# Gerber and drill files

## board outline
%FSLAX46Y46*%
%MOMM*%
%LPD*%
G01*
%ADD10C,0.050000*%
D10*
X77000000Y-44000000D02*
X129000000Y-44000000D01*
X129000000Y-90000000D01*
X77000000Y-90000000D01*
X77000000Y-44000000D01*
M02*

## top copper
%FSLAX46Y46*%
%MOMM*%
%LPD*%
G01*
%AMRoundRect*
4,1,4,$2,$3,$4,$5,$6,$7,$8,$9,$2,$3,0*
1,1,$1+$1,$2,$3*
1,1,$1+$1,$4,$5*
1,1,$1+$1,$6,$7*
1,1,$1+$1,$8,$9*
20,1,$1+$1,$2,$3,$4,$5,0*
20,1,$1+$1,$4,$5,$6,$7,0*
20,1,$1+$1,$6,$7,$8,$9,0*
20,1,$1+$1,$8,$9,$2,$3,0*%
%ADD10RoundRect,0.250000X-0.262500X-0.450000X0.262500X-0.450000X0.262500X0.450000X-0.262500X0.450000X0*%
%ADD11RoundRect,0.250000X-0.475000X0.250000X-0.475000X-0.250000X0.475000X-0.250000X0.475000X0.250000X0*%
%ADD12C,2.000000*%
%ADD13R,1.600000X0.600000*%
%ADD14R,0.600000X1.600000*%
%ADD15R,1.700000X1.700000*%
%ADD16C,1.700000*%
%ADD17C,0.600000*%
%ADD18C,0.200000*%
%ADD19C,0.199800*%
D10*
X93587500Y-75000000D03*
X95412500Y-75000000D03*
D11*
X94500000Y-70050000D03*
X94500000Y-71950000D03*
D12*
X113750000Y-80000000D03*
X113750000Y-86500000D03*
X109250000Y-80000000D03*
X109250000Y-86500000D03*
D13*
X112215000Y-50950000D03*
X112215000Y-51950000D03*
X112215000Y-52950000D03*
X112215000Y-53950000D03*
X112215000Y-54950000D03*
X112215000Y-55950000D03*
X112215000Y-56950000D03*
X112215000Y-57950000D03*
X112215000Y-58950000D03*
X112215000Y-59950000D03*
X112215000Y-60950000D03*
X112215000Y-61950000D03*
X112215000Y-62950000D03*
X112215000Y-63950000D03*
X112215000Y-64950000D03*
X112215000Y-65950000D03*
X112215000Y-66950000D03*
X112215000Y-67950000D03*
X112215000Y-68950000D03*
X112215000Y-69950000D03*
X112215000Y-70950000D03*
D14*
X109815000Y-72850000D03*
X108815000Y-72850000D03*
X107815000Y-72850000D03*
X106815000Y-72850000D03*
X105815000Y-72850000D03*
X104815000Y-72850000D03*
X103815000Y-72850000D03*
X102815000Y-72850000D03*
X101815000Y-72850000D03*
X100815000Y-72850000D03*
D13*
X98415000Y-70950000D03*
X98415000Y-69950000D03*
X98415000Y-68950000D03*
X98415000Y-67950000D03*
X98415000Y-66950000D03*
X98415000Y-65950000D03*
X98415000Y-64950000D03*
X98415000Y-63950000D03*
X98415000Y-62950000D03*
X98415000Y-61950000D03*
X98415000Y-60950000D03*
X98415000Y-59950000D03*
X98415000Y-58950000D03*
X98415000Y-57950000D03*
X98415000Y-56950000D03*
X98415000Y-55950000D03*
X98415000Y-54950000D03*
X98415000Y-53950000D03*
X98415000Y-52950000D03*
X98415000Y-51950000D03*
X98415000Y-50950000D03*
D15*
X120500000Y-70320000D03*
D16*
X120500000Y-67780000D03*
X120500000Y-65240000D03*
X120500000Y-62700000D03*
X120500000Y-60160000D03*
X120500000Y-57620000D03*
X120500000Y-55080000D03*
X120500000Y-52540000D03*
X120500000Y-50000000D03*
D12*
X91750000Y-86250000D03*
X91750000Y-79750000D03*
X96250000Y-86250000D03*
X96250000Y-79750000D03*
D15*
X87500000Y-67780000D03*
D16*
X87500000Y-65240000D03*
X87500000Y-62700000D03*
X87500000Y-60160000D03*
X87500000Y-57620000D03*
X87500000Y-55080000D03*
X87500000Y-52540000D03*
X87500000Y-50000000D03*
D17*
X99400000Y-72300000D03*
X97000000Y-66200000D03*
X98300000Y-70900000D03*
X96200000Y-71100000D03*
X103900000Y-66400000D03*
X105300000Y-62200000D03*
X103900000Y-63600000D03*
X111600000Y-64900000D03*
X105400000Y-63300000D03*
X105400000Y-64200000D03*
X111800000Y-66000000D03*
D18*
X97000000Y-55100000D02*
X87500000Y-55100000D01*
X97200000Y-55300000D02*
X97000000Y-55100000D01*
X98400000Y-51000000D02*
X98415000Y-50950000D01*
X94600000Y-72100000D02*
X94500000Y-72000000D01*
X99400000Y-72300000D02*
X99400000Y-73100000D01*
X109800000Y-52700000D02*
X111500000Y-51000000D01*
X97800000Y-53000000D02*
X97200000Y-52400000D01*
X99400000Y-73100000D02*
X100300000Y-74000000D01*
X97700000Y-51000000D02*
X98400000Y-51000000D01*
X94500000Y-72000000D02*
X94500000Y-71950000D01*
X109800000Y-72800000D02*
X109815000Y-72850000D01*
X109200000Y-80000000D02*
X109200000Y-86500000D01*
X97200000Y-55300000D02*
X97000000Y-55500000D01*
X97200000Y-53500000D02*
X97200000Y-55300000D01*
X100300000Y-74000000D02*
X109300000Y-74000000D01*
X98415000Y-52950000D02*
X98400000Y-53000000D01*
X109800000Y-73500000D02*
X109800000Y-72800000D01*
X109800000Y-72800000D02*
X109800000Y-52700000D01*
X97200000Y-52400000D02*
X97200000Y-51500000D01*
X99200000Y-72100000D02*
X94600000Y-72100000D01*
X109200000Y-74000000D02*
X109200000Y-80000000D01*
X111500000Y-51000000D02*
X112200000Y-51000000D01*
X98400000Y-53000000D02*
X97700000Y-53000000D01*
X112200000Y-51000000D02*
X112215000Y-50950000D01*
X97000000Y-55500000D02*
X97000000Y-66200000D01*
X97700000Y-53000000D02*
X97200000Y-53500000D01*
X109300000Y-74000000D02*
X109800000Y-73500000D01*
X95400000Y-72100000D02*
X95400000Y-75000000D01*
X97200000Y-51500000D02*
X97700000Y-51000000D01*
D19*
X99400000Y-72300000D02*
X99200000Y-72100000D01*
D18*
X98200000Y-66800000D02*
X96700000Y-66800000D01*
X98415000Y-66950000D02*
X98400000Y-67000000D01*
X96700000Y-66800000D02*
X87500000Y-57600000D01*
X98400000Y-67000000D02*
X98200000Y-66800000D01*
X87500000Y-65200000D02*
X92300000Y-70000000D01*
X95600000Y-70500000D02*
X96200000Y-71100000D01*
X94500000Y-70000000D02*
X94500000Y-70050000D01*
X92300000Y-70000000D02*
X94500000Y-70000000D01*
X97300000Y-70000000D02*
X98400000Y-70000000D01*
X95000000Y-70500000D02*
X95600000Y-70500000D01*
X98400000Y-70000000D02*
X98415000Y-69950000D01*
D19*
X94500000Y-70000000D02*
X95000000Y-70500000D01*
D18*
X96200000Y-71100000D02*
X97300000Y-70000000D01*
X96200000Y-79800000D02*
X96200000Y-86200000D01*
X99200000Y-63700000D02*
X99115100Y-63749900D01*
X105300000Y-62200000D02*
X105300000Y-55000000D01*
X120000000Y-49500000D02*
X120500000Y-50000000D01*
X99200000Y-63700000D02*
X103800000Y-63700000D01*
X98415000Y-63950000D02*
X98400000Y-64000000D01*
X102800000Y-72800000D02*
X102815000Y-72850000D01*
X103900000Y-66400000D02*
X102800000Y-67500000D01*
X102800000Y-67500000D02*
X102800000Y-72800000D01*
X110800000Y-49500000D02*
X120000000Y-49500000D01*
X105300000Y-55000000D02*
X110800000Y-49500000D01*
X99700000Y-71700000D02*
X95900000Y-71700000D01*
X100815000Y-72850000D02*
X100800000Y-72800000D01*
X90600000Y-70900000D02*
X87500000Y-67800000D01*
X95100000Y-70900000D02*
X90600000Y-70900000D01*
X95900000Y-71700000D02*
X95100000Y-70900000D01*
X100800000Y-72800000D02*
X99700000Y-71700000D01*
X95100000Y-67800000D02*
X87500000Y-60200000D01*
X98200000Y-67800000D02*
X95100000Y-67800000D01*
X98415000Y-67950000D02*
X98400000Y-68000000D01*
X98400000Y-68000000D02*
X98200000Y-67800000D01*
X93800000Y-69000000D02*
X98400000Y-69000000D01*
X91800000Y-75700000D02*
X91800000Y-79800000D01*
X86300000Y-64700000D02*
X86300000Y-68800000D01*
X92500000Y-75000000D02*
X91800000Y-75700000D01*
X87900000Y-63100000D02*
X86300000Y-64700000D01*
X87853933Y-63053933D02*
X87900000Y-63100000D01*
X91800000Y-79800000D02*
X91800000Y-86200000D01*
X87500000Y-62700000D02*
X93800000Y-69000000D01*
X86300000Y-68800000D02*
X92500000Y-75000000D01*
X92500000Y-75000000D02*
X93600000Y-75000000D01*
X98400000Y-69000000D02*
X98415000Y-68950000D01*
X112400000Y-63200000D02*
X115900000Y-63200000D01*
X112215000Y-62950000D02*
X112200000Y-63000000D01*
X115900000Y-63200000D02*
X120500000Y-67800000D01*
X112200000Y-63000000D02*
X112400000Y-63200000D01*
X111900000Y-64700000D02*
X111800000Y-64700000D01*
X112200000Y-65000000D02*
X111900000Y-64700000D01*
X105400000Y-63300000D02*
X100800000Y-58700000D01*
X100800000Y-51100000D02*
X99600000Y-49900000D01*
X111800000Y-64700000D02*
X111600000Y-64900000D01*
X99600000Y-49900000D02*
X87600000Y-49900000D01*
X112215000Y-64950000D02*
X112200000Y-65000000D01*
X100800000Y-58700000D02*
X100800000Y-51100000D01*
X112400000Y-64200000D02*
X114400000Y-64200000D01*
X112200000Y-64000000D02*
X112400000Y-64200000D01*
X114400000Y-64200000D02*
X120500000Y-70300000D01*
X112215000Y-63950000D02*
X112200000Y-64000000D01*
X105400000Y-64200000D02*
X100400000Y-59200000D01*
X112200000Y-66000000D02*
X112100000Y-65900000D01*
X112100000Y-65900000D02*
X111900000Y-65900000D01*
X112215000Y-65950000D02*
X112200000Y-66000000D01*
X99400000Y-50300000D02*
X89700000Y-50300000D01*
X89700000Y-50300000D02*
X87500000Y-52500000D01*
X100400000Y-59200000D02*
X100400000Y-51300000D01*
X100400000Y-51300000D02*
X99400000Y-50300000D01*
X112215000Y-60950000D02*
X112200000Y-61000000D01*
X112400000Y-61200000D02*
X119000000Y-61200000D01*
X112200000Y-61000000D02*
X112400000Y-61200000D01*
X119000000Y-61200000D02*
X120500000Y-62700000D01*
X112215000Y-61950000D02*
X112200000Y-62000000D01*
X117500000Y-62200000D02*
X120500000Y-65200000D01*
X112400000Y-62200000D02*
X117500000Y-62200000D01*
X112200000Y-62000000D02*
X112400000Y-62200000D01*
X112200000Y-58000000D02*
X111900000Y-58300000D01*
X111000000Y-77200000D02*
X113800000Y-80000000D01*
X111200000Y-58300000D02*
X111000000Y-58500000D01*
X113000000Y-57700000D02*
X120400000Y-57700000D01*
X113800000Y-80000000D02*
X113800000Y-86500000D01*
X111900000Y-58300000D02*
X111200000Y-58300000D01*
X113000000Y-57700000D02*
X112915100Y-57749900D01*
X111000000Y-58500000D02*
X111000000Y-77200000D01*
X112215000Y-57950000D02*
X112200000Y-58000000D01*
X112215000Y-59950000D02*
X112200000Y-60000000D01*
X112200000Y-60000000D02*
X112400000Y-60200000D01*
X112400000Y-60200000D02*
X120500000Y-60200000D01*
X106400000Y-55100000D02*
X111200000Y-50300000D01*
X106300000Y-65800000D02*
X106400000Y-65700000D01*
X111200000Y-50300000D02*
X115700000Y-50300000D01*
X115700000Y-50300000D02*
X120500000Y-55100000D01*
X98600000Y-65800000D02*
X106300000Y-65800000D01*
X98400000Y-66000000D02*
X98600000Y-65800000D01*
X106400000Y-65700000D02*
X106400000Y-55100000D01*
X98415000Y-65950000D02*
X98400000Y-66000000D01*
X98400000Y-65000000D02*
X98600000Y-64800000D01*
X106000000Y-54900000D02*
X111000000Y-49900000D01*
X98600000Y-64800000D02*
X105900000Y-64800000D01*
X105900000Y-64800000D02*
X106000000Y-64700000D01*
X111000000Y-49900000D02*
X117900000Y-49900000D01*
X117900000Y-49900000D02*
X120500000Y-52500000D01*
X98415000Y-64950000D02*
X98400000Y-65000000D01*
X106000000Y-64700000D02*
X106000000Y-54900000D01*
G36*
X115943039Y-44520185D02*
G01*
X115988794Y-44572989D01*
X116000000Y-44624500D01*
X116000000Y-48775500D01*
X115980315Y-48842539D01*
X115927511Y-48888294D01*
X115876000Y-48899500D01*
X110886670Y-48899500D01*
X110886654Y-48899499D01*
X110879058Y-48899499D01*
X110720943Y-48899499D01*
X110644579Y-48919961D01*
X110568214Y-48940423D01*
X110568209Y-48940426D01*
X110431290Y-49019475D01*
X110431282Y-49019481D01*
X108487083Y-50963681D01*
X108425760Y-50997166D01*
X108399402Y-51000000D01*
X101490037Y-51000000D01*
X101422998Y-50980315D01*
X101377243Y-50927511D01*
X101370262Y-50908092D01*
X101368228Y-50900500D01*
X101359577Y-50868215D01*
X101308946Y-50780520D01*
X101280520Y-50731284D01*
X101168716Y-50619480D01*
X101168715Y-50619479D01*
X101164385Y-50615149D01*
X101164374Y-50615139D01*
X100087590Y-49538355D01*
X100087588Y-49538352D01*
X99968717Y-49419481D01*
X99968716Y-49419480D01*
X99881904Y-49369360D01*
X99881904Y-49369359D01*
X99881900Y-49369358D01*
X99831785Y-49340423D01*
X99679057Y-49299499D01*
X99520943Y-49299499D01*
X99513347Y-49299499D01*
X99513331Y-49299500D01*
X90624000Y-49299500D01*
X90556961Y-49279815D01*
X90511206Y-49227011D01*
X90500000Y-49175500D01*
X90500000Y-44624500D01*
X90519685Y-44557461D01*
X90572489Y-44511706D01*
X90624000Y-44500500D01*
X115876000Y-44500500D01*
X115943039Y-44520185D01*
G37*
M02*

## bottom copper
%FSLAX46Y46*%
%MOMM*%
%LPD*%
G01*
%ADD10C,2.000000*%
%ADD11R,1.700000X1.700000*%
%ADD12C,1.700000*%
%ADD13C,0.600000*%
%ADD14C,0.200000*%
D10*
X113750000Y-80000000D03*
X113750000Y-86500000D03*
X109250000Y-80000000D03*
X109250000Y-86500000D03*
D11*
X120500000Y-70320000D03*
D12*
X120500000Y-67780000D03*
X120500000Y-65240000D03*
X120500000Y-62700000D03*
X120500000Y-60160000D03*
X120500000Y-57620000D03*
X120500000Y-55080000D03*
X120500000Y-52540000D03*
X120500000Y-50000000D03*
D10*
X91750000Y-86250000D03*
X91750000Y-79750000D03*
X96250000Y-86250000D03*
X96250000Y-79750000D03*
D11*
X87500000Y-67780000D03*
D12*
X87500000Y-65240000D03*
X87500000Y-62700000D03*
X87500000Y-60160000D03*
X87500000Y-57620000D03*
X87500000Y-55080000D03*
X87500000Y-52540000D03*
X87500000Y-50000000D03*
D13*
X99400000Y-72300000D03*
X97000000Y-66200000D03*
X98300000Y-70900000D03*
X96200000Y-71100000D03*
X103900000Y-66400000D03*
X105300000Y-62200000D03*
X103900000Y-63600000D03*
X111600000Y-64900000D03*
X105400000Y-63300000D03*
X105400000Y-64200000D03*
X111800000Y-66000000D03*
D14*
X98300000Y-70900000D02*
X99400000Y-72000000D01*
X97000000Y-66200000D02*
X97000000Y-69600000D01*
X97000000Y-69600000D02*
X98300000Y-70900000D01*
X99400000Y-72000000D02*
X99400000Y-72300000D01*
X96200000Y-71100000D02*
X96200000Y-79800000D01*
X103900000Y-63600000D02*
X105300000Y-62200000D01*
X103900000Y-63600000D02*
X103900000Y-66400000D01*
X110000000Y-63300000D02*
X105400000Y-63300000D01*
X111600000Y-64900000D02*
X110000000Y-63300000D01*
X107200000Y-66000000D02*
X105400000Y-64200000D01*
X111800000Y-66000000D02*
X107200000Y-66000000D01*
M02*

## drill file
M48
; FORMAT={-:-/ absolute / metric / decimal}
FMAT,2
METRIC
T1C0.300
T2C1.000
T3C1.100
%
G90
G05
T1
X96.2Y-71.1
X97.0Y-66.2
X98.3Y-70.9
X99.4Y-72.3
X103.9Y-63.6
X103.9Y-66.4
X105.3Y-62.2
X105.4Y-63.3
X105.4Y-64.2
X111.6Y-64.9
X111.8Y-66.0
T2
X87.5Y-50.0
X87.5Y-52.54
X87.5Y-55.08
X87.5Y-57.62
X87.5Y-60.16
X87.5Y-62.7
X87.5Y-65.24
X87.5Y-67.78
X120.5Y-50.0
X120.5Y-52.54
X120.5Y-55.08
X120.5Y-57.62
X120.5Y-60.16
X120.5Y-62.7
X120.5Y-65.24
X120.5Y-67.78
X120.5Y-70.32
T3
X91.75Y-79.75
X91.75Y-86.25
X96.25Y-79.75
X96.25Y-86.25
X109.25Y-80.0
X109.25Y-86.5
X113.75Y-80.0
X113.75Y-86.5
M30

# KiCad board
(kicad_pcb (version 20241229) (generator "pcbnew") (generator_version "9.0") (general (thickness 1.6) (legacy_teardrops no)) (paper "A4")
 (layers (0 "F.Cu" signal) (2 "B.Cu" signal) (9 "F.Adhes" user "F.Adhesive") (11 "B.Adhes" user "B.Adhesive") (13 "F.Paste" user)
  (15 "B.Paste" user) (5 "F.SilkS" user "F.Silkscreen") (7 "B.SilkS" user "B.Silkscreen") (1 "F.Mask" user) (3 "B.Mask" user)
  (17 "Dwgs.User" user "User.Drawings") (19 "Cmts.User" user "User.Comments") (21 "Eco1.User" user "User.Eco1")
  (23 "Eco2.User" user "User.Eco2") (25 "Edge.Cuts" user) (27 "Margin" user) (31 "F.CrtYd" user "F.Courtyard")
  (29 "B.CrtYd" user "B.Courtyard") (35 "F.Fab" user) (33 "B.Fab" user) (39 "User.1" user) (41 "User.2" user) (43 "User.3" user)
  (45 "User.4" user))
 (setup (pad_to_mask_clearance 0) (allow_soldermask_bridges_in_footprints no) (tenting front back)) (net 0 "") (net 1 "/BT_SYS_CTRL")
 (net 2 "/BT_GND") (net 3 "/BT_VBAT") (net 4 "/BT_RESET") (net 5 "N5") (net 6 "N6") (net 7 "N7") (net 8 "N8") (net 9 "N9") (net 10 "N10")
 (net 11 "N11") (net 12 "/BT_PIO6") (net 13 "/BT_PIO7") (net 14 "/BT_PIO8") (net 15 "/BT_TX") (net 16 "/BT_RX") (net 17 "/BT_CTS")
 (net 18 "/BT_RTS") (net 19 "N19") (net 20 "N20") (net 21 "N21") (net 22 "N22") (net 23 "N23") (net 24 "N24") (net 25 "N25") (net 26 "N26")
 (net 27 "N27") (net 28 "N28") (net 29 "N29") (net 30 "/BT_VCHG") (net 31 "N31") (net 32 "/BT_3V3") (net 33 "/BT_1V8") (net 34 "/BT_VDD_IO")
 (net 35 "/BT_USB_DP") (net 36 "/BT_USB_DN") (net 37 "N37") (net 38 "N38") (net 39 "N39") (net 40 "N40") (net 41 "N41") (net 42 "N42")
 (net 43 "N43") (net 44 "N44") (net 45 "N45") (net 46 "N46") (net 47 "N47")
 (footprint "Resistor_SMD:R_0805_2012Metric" (layer "F.Cu") (at 94.5 75)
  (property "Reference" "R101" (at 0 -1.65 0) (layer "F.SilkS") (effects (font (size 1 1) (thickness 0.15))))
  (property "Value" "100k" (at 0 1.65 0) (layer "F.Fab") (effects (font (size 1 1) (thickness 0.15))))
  (pad "1" smd roundrect (at -0.9125 0) (size 1.025 1.4) (layers "F.Cu" "F.Mask" "F.Paste") (roundrect_rratio 0.243902)
   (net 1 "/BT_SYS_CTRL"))
  (pad "2" smd roundrect (at 0.9125 0) (size 1.025 1.4) (layers "F.Cu" "F.Mask" "F.Paste") (roundrect_rratio 0.243902) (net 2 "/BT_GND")))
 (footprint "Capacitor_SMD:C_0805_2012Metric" (layer "F.Cu") (at 94.5 71 -90)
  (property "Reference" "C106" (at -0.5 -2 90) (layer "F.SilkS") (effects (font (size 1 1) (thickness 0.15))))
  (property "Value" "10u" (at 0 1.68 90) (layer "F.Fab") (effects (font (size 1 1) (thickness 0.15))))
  (pad "1" smd roundrect (at -0.95 0 270) (size 1 1.45) (layers "F.Cu" "F.Mask" "F.Paste") (roundrect_rratio 0.25) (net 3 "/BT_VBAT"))
  (pad "2" smd roundrect (at 0.95 0 270) (size 1 1.45) (layers "F.Cu" "F.Mask" "F.Paste") (roundrect_rratio 0.25) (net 2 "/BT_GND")))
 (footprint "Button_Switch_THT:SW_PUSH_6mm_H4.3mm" (layer "F.Cu") (at 113.75 80 -90)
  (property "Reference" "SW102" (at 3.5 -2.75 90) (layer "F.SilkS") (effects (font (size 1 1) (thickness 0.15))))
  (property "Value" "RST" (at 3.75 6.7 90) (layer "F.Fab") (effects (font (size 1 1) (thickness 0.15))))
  (pad "1" thru_hole circle (at 0 0) (size 2 2) (drill 1.1) (layers "*.Cu" "*.Mask") (remove_unused_layers no) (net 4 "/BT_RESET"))
  (pad "1" thru_hole circle (at 6.5 0) (size 2 2) (drill 1.1) (layers "*.Cu" "*.Mask") (remove_unused_layers no) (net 4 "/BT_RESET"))
  (pad "2" thru_hole circle (at 0 4.5) (size 2 2) (drill 1.1) (layers "*.Cu" "*.Mask") (remove_unused_layers no) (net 2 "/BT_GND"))
  (pad "2" thru_hole circle (at 6.5 4.5) (size 2 2) (drill 1.1) (layers "*.Cu" "*.Mask") (remove_unused_layers no) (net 2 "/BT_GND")))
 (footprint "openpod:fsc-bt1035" (layer "F.Cu") (at 105.315 59 180)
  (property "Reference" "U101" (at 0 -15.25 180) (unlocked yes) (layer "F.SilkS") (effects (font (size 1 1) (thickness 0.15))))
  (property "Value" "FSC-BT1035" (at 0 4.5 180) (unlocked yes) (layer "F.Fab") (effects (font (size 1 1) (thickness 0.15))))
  (pad "1" smd rect (at -6.9 8.05 180) (size 1.6 0.6) (layers "F.Cu" "F.Mask" "F.Paste") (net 2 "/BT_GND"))
  (pad "2" smd rect (at -6.9 7.05 180) (size 1.6 0.6) (layers "F.Cu" "F.Mask" "F.Paste") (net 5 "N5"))
  (pad "3" smd rect (at -6.9 6.05 180) (size 1.6 0.6) (layers "F.Cu" "F.Mask" "F.Paste") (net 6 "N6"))
  (pad "4" smd rect (at -6.9 5.05 180) (size 1.6 0.6) (layers "F.Cu" "F.Mask" "F.Paste") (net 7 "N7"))
  (pad "5" smd rect (at -6.9 4.05 180) (size 1.6 0.6) (layers "F.Cu" "F.Mask" "F.Paste") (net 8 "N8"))
  (pad "6" smd rect (at -6.9 3.05 180) (size 1.6 0.6) (layers "F.Cu" "F.Mask" "F.Paste") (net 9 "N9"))
  (pad "7" smd rect (at -6.9 2.05 180) (size 1.6 0.6) (layers "F.Cu" "F.Mask" "F.Paste") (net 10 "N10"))
  (pad "8" smd rect (at -6.9 1.05 180) (size 1.6 0.6) (layers "F.Cu" "F.Mask" "F.Paste") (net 4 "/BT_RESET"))
  (pad "9" smd rect (at -6.9 0.05 180) (size 1.6 0.6) (layers "F.Cu" "F.Mask" "F.Paste") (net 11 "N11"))
  (pad "10" smd rect (at -6.9 -0.95 180) (size 1.6 0.6) (layers "F.Cu" "F.Mask" "F.Paste") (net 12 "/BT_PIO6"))
  (pad "11" smd rect (at -6.9 -1.95 180) (size 1.6 0.6) (layers "F.Cu" "F.Mask" "F.Paste") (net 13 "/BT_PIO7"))
  (pad "12" smd rect (at -6.9 -2.95 180) (size 1.6 0.6) (layers "F.Cu" "F.Mask" "F.Paste") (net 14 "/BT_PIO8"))
  (pad "13" smd rect (at -6.9 -3.95 180) (size 1.6 0.6) (layers "F.Cu" "F.Mask" "F.Paste") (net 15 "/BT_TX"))
  (pad "14" smd rect (at -6.9 -4.95 180) (size 1.6 0.6) (layers "F.Cu" "F.Mask" "F.Paste") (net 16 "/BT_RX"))
  (pad "15" smd rect (at -6.9 -5.95 180) (size 1.6 0.6) (layers "F.Cu" "F.Mask" "F.Paste") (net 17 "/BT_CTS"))
  (pad "16" smd rect (at -6.9 -6.95 180) (size 1.6 0.6) (layers "F.Cu" "F.Mask" "F.Paste") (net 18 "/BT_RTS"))
  (pad "17" smd rect (at -6.9 -7.95 180) (size 1.6 0.6) (layers "F.Cu" "F.Mask" "F.Paste") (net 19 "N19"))
  (pad "18" smd rect (at -6.9 -8.95 180) (size 1.6 0.6) (layers "F.Cu" "F.Mask" "F.Paste") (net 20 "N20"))
  (pad "19" smd rect (at -6.9 -9.95 180) (size 1.6 0.6) (layers "F.Cu" "F.Mask" "F.Paste") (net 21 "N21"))
  (pad "20" smd rect (at -6.9 -10.95 180) (size 1.6 0.6) (layers "F.Cu" "F.Mask" "F.Paste") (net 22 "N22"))
  (pad "21" smd rect (at -6.9 -11.95 180) (size 1.6 0.6) (layers "F.Cu" "F.Mask" "F.Paste") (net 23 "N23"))
  (pad "22" smd rect (at -4.5 -13.85 180) (size 0.6 1.6) (layers "F.Cu" "F.Mask" "F.Paste") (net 2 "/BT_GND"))
  (pad "23" smd rect (at -3.5 -13.85 180) (size 0.6 1.6) (layers "F.Cu" "F.Mask" "F.Paste") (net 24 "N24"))
  (pad "24" smd rect (at -2.5 -13.85 180) (size 0.6 1.6) (layers "F.Cu" "F.Mask" "F.Paste") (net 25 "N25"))
  (pad "25" smd rect (at -1.5 -13.85 180) (size 0.6 1.6) (layers "F.Cu" "F.Mask" "F.Paste") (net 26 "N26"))
  (pad "26" smd rect (at -0.5 -13.85 180) (size 0.6 1.6) (layers "F.Cu" "F.Mask" "F.Paste") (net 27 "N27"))
  (pad "27" smd rect (at 0.5 -13.85 180) (size 0.6 1.6) (layers "F.Cu" "F.Mask" "F.Paste") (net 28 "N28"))
  (pad "28" smd rect (at 1.5 -13.85 180) (size 0.6 1.6) (layers "F.Cu" "F.Mask" "F.Paste") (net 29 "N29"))
  (pad "29" smd rect (at 2.5 -13.85 180) (size 0.6 1.6) (layers "F.Cu" "F.Mask" "F.Paste") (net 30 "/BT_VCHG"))
  (pad "30" smd rect (at 3.5 -13.85 180) (size 0.6 1.6) (layers "F.Cu" "F.Mask" "F.Paste") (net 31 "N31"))
  (pad "31" smd rect (at 4.5 -13.85 180) (size 0.6 1.6) (layers "F.Cu" "F.Mask" "F.Paste") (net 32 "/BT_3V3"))
  (pad "32" smd rect (at 6.9 -11.95 180) (size 1.6 0.6) (layers "F.Cu" "F.Mask" "F.Paste") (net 2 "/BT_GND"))
  (pad "33" smd rect (at 6.9 -10.95 180) (size 1.6 0.6) (layers "F.Cu" "F.Mask" "F.Paste") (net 3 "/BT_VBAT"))
  (pad "34" smd rect (at 6.9 -9.95 180) (size 1.6 0.6) (layers "F.Cu" "F.Mask" "F.Paste") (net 1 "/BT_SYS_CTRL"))
  (pad "35" smd rect (at 6.9 -8.95 180) (size 1.6 0.6) (layers "F.Cu" "F.Mask" "F.Paste") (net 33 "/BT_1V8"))
  (pad "36" smd rect (at 6.9 -7.95 180) (size 1.6 0.6) (layers "F.Cu" "F.Mask" "F.Paste") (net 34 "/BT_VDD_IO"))
  (pad "37" smd rect (at 6.9 -6.95 180) (size 1.6 0.6) (layers "F.Cu" "F.Mask" "F.Paste") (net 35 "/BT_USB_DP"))
  (pad "38" smd rect (at 6.9 -5.95 180) (size 1.6 0.6) (layers "F.Cu" "F.Mask" "F.Paste") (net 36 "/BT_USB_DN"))
  (pad "39" smd rect (at 6.9 -4.95 180) (size 1.6 0.6) (layers "F.Cu" "F.Mask" "F.Paste") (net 30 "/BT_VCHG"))
  (pad "40" smd rect (at 6.9 -3.95 180) (size 1.6 0.6) (layers "F.Cu" "F.Mask" "F.Paste") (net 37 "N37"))
  (pad "41" smd rect (at 6.9 -2.95 180) (size 1.6 0.6) (layers "F.Cu" "F.Mask" "F.Paste") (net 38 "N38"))
  (pad "42" smd rect (at 6.9 -1.95 180) (size 1.6 0.6) (layers "F.Cu" "F.Mask" "F.Paste") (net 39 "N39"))
  (pad "43" smd rect (at 6.9 -0.95 180) (size 1.6 0.6) (layers "F.Cu" "F.Mask" "F.Paste") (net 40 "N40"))
  (pad "44" smd rect (at 6.9 0.05 180) (size 1.6 0.6) (layers "F.Cu" "F.Mask" "F.Paste") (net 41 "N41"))
  (pad "45" smd rect (at 6.9 1.05 180) (size 1.6 0.6) (layers "F.Cu" "F.Mask" "F.Paste") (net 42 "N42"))
  (pad "46" smd rect (at 6.9 2.05 180) (size 1.6 0.6) (layers "F.Cu" "F.Mask" "F.Paste") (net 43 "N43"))
  (pad "47" smd rect (at 6.9 3.05 180) (size 1.6 0.6) (layers "F.Cu" "F.Mask" "F.Paste") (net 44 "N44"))
  (pad "48" smd rect (at 6.9 4.05 180) (size 1.6 0.6) (layers "F.Cu" "F.Mask" "F.Paste") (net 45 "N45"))
  (pad "49" smd rect (at 6.9 5.05 180) (size 1.6 0.6) (layers "F.Cu" "F.Mask" "F.Paste") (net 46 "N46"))
  (pad "50" smd rect (at 6.9 6.05 180) (size 1.6 0.6) (layers "F.Cu" "F.Mask" "F.Paste") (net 2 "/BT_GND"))
  (pad "51" smd rect (at 6.9 7.05 180) (size 1.6 0.6) (layers "F.Cu" "F.Mask" "F.Paste") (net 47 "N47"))
  (pad "52" smd rect (at 6.9 8.05 180) (size 1.6 0.6) (layers "F.Cu" "F.Mask" "F.Paste") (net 2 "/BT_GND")))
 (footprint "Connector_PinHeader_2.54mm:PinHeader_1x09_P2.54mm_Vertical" (layer "F.Cu") (at 120.5 70.32 180)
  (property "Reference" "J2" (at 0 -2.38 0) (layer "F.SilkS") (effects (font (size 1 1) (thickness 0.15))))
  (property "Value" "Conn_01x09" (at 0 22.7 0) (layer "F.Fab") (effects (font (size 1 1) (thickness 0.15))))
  (pad "1" thru_hole rect (at 0 0 180) (size 1.7 1.7) (drill 1) (layers "*.Cu" "*.Mask") (remove_unused_layers no) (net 16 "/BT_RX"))
  (pad "2" thru_hole circle (at 0 2.54 180) (size 1.7 1.7) (drill 1) (layers "*.Cu" "*.Mask") (remove_unused_layers no) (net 15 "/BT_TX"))
  (pad "3" thru_hole circle (at 0 5.08 180) (size 1.7 1.7) (drill 1) (layers "*.Cu" "*.Mask") (remove_unused_layers no) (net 14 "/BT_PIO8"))
  (pad "4" thru_hole circle (at 0 7.62 180) (size 1.7 1.7) (drill 1) (layers "*.Cu" "*.Mask") (remove_unused_layers no) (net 13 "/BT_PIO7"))
  (pad "5" thru_hole circle (at 0 10.16 180) (size 1.7 1.7) (drill 1) (layers "*.Cu" "*.Mask") (remove_unused_layers no) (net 12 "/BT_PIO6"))
  (pad "6" thru_hole circle (at 0 12.7 180) (size 1.7 1.7) (drill 1) (layers "*.Cu" "*.Mask") (remove_unused_layers no) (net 4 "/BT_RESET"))
  (pad "7" thru_hole circle (at 0 15.24 180) (size 1.7 1.7) (drill 1) (layers "*.Cu" "*.Mask") (remove_unused_layers no)
   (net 35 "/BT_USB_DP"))
  (pad "8" thru_hole circle (at 0 17.78 180) (size 1.7 1.7) (drill 1) (layers "*.Cu" "*.Mask") (remove_unused_layers no)
   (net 36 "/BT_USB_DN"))
  (pad "9" thru_hole circle (at 0 20.32 180) (size 1.7 1.7) (drill 1) (layers "*.Cu" "*.Mask") (remove_unused_layers no) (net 30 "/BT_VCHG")))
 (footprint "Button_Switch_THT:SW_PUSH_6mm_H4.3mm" (layer "F.Cu") (at 91.75 86.25 90)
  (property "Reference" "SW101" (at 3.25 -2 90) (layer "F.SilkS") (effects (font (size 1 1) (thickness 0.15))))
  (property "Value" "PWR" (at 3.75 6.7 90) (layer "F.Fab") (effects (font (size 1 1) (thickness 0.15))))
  (pad "1" thru_hole circle (at 0 0 180) (size 2 2) (drill 1.1) (layers "*.Cu" "*.Mask") (remove_unused_layers no) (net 1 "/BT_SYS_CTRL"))
  (pad "1" thru_hole circle (at 6.5 0 180) (size 2 2) (drill 1.1) (layers "*.Cu" "*.Mask") (remove_unused_layers no) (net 1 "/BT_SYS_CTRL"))
  (pad "2" thru_hole circle (at 0 4.5 180) (size 2 2) (drill 1.1) (layers "*.Cu" "*.Mask") (remove_unused_layers no) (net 3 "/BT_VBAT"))
  (pad "2" thru_hole circle (at 6.5 4.5 180) (size 2 2) (drill 1.1) (layers "*.Cu" "*.Mask") (remove_unused_layers no) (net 3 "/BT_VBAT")))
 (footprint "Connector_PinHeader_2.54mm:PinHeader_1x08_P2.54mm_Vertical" (layer "F.Cu") (at 87.5 67.78 180)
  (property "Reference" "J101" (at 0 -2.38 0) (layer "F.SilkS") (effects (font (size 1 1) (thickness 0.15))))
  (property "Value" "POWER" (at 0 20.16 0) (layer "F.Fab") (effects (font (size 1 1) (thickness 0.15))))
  (pad "1" thru_hole rect (at 0 0 180) (size 1.7 1.7) (drill 1) (layers "*.Cu" "*.Mask") (remove_unused_layers no) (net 32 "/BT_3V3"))
  (pad "2" thru_hole circle (at 0 2.54 180) (size 1.7 1.7) (drill 1) (layers "*.Cu" "*.Mask") (remove_unused_layers no) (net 3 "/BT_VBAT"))
  (pad "3" thru_hole circle (at 0 5.08 180) (size 1.7 1.7) (drill 1) (layers "*.Cu" "*.Mask") (remove_unused_layers no)
   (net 1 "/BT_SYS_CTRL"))
  (pad "4" thru_hole circle (at 0 7.62 180) (size 1.7 1.7) (drill 1) (layers "*.Cu" "*.Mask") (remove_unused_layers no) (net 33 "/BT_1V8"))
  (pad "5" thru_hole circle (at 0 10.16 180) (size 1.7 1.7) (drill 1) (layers "*.Cu" "*.Mask") (remove_unused_layers no)
   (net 34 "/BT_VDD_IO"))
  (pad "6" thru_hole circle (at 0 12.7 180) (size 1.7 1.7) (drill 1) (layers "*.Cu" "*.Mask") (remove_unused_layers no) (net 2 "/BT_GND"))
  (pad "7" thru_hole circle (at 0 15.24 180) (size 1.7 1.7) (drill 1) (layers "*.Cu" "*.Mask") (remove_unused_layers no) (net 18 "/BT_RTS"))
  (pad "8" thru_hole circle (at 0 17.78 180) (size 1.7 1.7) (drill 1) (layers "*.Cu" "*.Mask") (remove_unused_layers no) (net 17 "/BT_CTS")))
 (gr_rect (start 77 44) (end 129 90) (stroke (width 0.05) (type default)) (fill no) (layer "Edge.Cuts"))
 (segment (start 97 55.1) (end 87.5 55.1) (width 0.2) (layer "F.Cu") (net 2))
 (segment (start 97.2 55.3) (end 97 55.1) (width 0.2) (layer "F.Cu") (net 2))
 (segment (start 98.4 51) (end 98.415 50.95) (width 0.2) (layer "F.Cu") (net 2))
 (segment (start 94.6 72.1) (end 94.5 72) (width 0.2) (layer "F.Cu") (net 2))
 (segment (start 99.4 72.3) (end 99.4 73.1) (width 0.2) (layer "F.Cu") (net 2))
 (segment (start 109.8 52.7) (end 111.5 51) (width 0.2) (layer "F.Cu") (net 2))
 (segment (start 97.8 53) (end 97.2 52.4) (width 0.2) (layer "F.Cu") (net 2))
 (segment (start 99.4 73.1) (end 100.3 74) (width 0.2) (layer "F.Cu") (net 2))
 (segment (start 97.7 51) (end 98.4 51) (width 0.2) (layer "F.Cu") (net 2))
 (segment (start 94.5 72) (end 94.5 71.95) (width 0.2) (layer "F.Cu") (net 2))
 (segment (start 109.8 72.8) (end 109.815 72.85) (width 0.2) (layer "F.Cu") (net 2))
 (segment (start 109.2 80) (end 109.2 86.5) (width 0.2) (layer "F.Cu") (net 2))
 (segment (start 97.2 55.3) (end 97 55.5) (width 0.2) (layer "F.Cu") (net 2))
 (segment (start 97.2 53.5) (end 97.2 55.3) (width 0.2) (layer "F.Cu") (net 2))
 (segment (start 100.3 74) (end 109.3 74) (width 0.2) (layer "F.Cu") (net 2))
 (segment (start 98.415 52.95) (end 98.4 53) (width 0.2) (layer "F.Cu") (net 2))
 (segment (start 109.8 73.5) (end 109.8 72.8) (width 0.2) (layer "F.Cu") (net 2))
 (segment (start 109.8 72.8) (end 109.8 52.7) (width 0.2) (layer "F.Cu") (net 2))
 (segment (start 97.2 52.4) (end 97.2 51.5) (width 0.2) (layer "F.Cu") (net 2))
 (segment (start 99.2 72.1) (end 94.6 72.1) (width 0.2) (layer "F.Cu") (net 2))
 (segment (start 109.2 74) (end 109.2 80) (width 0.2) (layer "F.Cu") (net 2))
 (segment (start 111.5 51) (end 112.2 51) (width 0.2) (layer "F.Cu") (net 2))
 (segment (start 98.4 53) (end 97.7 53) (width 0.2) (layer "F.Cu") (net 2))
 (segment (start 112.2 51) (end 112.215 50.95) (width 0.2) (layer "F.Cu") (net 2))
 (segment (start 97 55.5) (end 97 66.2) (width 0.2) (layer "F.Cu") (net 2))
 (segment (start 97.7 53) (end 97.2 53.5) (width 0.2) (layer "F.Cu") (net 2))
 (segment (start 109.3 74) (end 109.8 73.5) (width 0.2) (layer "F.Cu") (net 2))
 (segment (start 95.4 72.1) (end 95.4 75) (width 0.2) (layer "F.Cu") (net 2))
 (segment (start 97.2 51.5) (end 97.7 51) (width 0.2) (layer "F.Cu") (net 2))
 (segment (start 99.4 72.3) (end 99.2 72.1) (width 0.1998) (layer "F.Cu") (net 2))
 (via (at 99.4 72.3) (size 0.6) (drill 0.3) (layers "F.Cu" "B.Cu") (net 2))
 (via (at 97 66.2) (size 0.6) (drill 0.3) (layers "F.Cu" "B.Cu") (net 2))
 (via (at 98.3 70.9) (size 0.6) (drill 0.3) (layers "F.Cu" "B.Cu") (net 2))
 (segment (start 98.3 70.9) (end 99.4 72) (width 0.2) (layer "B.Cu") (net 2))
 (segment (start 97 66.2) (end 97 69.6) (width 0.2) (layer "B.Cu") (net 2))
 (segment (start 97 69.6) (end 98.3 70.9) (width 0.2) (layer "B.Cu") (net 2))
 (segment (start 99.4 72) (end 99.4 72.3) (width 0.2) (layer "B.Cu") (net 2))
 (segment (start 98.2 66.8) (end 96.7 66.8) (width 0.2) (layer "F.Cu") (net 34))
 (segment (start 98.415 66.95) (end 98.4 67) (width 0.2) (layer "F.Cu") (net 34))
 (segment (start 96.7 66.8) (end 87.5 57.6) (width 0.2) (layer "F.Cu") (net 34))
 (segment (start 98.4 67) (end 98.2 66.8) (width 0.2) (layer "F.Cu") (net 34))
 (segment (start 87.5 65.2) (end 92.3 70) (width 0.2) (layer "F.Cu") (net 3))
 (segment (start 95.6 70.5) (end 96.2 71.1) (width 0.2) (layer "F.Cu") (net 3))
 (segment (start 94.5 70) (end 94.5 70.05) (width 0.2) (layer "F.Cu") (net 3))
 (segment (start 92.3 70) (end 94.5 70) (width 0.2) (layer "F.Cu") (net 3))
 (segment (start 97.3 70) (end 98.4 70) (width 0.2) (layer "F.Cu") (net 3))
 (segment (start 95 70.5) (end 95.6 70.5) (width 0.2) (layer "F.Cu") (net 3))
 (segment (start 98.4 70) (end 98.415 69.95) (width 0.2) (layer "F.Cu") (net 3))
 (segment (start 94.5 70) (end 95 70.5) (width 0.1998) (layer "F.Cu") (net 3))
 (segment (start 96.2 71.1) (end 97.3 70) (width 0.2) (layer "F.Cu") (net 3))
 (segment (start 96.2 79.8) (end 96.2 86.2) (width 0.2) (layer "F.Cu") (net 3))
 (via (at 96.2 71.1) (size 0.6) (drill 0.3) (layers "F.Cu" "B.Cu") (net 3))
 (segment (start 96.2 71.1) (end 96.2 79.8) (width 0.2) (layer "B.Cu") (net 3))
 (segment (start 99.2 63.7) (end 99.1151 63.7499) (width 0.2) (layer "F.Cu") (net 30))
 (segment (start 105.3 62.2) (end 105.3 55) (width 0.2) (layer "F.Cu") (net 30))
 (segment (start 120 49.5) (end 120.5 50) (width 0.2) (layer "F.Cu") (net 30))
 (segment (start 99.2 63.7) (end 103.8 63.7) (width 0.2) (layer "F.Cu") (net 30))
 (segment (start 98.415 63.95) (end 98.4 64) (width 0.2) (layer "F.Cu") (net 30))
 (segment (start 102.8 72.8) (end 102.815 72.85) (width 0.2) (layer "F.Cu") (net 30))
 (segment (start 103.9 66.4) (end 102.8 67.5) (width 0.2) (layer "F.Cu") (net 30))
 (segment (start 102.8 67.5) (end 102.8 72.8) (width 0.2) (layer "F.Cu") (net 30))
 (segment (start 110.8 49.5) (end 120 49.5) (width 0.2) (layer "F.Cu") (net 30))
 (segment (start 105.3 55) (end 110.8 49.5) (width 0.2) (layer "F.Cu") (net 30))
 (via (at 103.9 66.4) (size 0.6) (drill 0.3) (layers "F.Cu" "B.Cu") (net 30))
 (via (at 105.3 62.2) (size 0.6) (drill 0.3) (layers "F.Cu" "B.Cu") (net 30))
 (via (at 103.9 63.6) (size 0.6) (drill 0.3) (layers "F.Cu" "B.Cu") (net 30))
 (segment (start 103.9 63.6) (end 105.3 62.2) (width 0.2) (layer "B.Cu") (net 30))
 (segment (start 103.9 63.6) (end 103.9 66.4) (width 0.2) (layer "B.Cu") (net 30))
 (segment (start 99.7 71.7) (end 95.9 71.7) (width 0.2) (layer "F.Cu") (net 32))
 (segment (start 100.815 72.85) (end 100.8 72.8) (width 0.2) (layer "F.Cu") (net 32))
 (segment (start 90.6 70.9) (end 87.5 67.8) (width 0.2) (layer "F.Cu") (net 32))
 (segment (start 95.1 70.9) (end 90.6 70.9) (width 0.2) (layer "F.Cu") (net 32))
 (segment (start 95.9 71.7) (end 95.1 70.9) (width 0.2) (layer "F.Cu") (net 32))
 (segment (start 100.8 72.8) (end 99.7 71.7) (width 0.2) (layer "F.Cu") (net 32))
 (segment (start 95.1 67.8) (end 87.5 60.2) (width 0.2) (layer "F.Cu") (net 33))
 (segment (start 98.2 67.8) (end 95.1 67.8) (width 0.2) (layer "F.Cu") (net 33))
 (segment (start 98.415 67.95) (end 98.4 68) (width 0.2) (layer "F.Cu") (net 33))
 (segment (start 98.4 68) (end 98.2 67.8) (width 0.2) (layer "F.Cu") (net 33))
 (segment (start 93.8 69) (end 98.4 69) (width 0.2) (layer "F.Cu") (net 1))
 (segment (start 91.8 75.7) (end 91.8 79.8) (width 0.2) (layer "F.Cu") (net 1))
 (segment (start 86.3 64.7) (end 86.3 68.8) (width 0.2) (layer "F.Cu") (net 1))
 (segment (start 92.5 75) (end 91.8 75.7) (width 0.2) (layer "F.Cu") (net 1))
 (segment (start 87.9 63.1) (end 86.3 64.7) (width 0.2) (layer "F.Cu") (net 1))
 (segment (start 87.853933 63.053933) (end 87.9 63.1) (width 0.2) (layer "F.Cu") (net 1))
 (segment (start 91.8 79.8) (end 91.8 86.2) (width 0.2) (layer "F.Cu") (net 1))
 (segment (start 87.5 62.7) (end 93.8 69) (width 0.2) (layer "F.Cu") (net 1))
 (segment (start 86.3 68.8) (end 92.5 75) (width 0.2) (layer "F.Cu") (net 1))
 (segment (start 92.5 75) (end 93.6 75) (width 0.2) (layer "F.Cu") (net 1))
 (segment (start 98.4 69) (end 98.415 68.95) (width 0.2) (layer "F.Cu") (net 1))
 (segment (start 112.4 63.2) (end 115.9 63.2) (width 0.2) (layer "F.Cu") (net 15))
 (segment (start 112.215 62.95) (end 112.2 63) (width 0.2) (layer "F.Cu") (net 15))
 (segment (start 115.9 63.2) (end 120.5 67.8) (width 0.2) (layer "F.Cu") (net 15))
 (segment (start 112.2 63) (end 112.4 63.2) (width 0.2) (layer "F.Cu") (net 15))
 (segment (start 111.9 64.7) (end 111.8 64.7) (width 0.2) (layer "F.Cu") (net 17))
 (segment (start 112.2 65) (end 111.9 64.7) (width 0.2) (layer "F.Cu") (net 17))
 (segment (start 105.4 63.3) (end 100.8 58.7) (width 0.2) (layer "F.Cu") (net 17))
 (segment (start 100.8 51.1) (end 99.6 49.9) (width 0.2) (layer "F.Cu") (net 17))
 (segment (start 111.8 64.7) (end 111.6 64.9) (width 0.2) (layer "F.Cu") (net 17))
 (segment (start 99.6 49.9) (end 87.6 49.9) (width 0.2) (layer "F.Cu") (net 17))
 (segment (start 112.215 64.95) (end 112.2 65) (width 0.2) (layer "F.Cu") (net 17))
 (segment (start 100.8 58.7) (end 100.8 51.1) (width 0.2) (layer "F.Cu") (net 17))
 (via (at 111.6 64.9) (size 0.6) (drill 0.3) (layers "F.Cu" "B.Cu") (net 17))
 (via (at 105.4 63.3) (size 0.6) (drill 0.3) (layers "F.Cu" "B.Cu") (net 17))
 (segment (start 110 63.3) (end 105.4 63.3) (width 0.2) (layer "B.Cu") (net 17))
 (segment (start 111.6 64.9) (end 110 63.3) (width 0.2) (layer "B.Cu") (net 17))
 (segment (start 112.4 64.2) (end 114.4 64.2) (width 0.2) (layer "F.Cu") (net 16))
 (segment (start 112.2 64) (end 112.4 64.2) (width 0.2) (layer "F.Cu") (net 16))
 (segment (start 114.4 64.2) (end 120.5 70.3) (width 0.2) (layer "F.Cu") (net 16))
 (segment (start 112.215 63.95) (end 112.2 64) (width 0.2) (layer "F.Cu") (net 16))
 (segment (start 105.4 64.2) (end 100.4 59.2) (width 0.2) (layer "F.Cu") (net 18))
 (segment (start 112.2 66) (end 112.1 65.9) (width 0.2) (layer "F.Cu") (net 18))
 (segment (start 112.1 65.9) (end 111.9 65.9) (width 0.2) (layer "F.Cu") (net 18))
 (segment (start 112.215 65.95) (end 112.2 66) (width 0.2) (layer "F.Cu") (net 18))
 (segment (start 99.4 50.3) (end 89.7 50.3) (width 0.2) (layer "F.Cu") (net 18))
 (segment (start 89.7 50.3) (end 87.5 52.5) (width 0.2) (layer "F.Cu") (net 18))
 (segment (start 100.4 59.2) (end 100.4 51.3) (width 0.2) (layer "F.Cu") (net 18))
 (segment (start 100.4 51.3) (end 99.4 50.3) (width 0.2) (layer "F.Cu") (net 18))
 (via (at 105.4 64.2) (size 0.6) (drill 0.3) (layers "F.Cu" "B.Cu") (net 18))
 (via (at 111.8 66) (size 0.6) (drill 0.3) (layers "F.Cu" "B.Cu") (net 18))
 (segment (start 107.2 66) (end 105.4 64.2) (width 0.2) (layer "B.Cu") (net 18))
 (segment (start 111.8 66) (end 107.2 66) (width 0.2) (layer "B.Cu") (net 18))
 (segment (start 112.215 60.95) (end 112.2 61) (width 0.2) (layer "F.Cu") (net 13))
 (segment (start 112.4 61.2) (end 119 61.2) (width 0.2) (layer "F.Cu") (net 13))
 (segment (start 112.2 61) (end 112.4 61.2) (width 0.2) (layer "F.Cu") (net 13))
 (segment (start 119 61.2) (end 120.5 62.7) (width 0.2) (layer "F.Cu") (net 13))
 (segment (start 112.215 61.95) (end 112.2 62) (width 0.2) (layer "F.Cu") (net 14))
 (segment (start 117.5 62.2) (end 120.5 65.2) (width 0.2) (layer "F.Cu") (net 14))
 (segment (start 112.4 62.2) (end 117.5 62.2) (width 0.2) (layer "F.Cu") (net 14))
 (segment (start 112.2 62) (end 112.4 62.2) (width 0.2) (layer "F.Cu") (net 14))
 (segment (start 112.2 58) (end 111.9 58.3) (width 0.2) (layer "F.Cu") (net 4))
 (segment (start 111 77.2) (end 113.8 80) (width 0.2) (layer "F.Cu") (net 4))
 (segment (start 111.2 58.3) (end 111 58.5) (width 0.2) (layer "F.Cu") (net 4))
 (segment (start 113 57.7) (end 120.4 57.7) (width 0.2) (layer "F.Cu") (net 4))
 (segment (start 113.8 80) (end 113.8 86.5) (width 0.2) (layer "F.Cu") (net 4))
 (segment (start 111.9 58.3) (end 111.2 58.3) (width 0.2) (layer "F.Cu") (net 4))
 (segment (start 113 57.7) (end 112.9151 57.7499) (width 0.2) (layer "F.Cu") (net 4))
 (segment (start 111 58.5) (end 111 77.2) (width 0.2) (layer "F.Cu") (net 4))
 (segment (start 112.215 57.95) (end 112.2 58) (width 0.2) (layer "F.Cu") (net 4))
 (segment (start 112.215 59.95) (end 112.2 60) (width 0.2) (layer "F.Cu") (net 12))
 (segment (start 112.2 60) (end 112.4 60.2) (width 0.2) (layer "F.Cu") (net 12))
 (segment (start 112.4 60.2) (end 120.5 60.2) (width 0.2) (layer "F.Cu") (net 12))
 (segment (start 106.4 55.1) (end 111.2 50.3) (width 0.2) (layer "F.Cu") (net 35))
 (segment (start 106.3 65.8) (end 106.4 65.7) (width 0.2) (layer "F.Cu") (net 35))
 (segment (start 111.2 50.3) (end 115.7 50.3) (width 0.2) (layer "F.Cu") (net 35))
 (segment (start 115.7 50.3) (end 120.5 55.1) (width 0.2) (layer "F.Cu") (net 35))
 (segment (start 98.6 65.8) (end 106.3 65.8) (width 0.2) (layer "F.Cu") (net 35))
 (segment (start 98.4 66) (end 98.6 65.8) (width 0.2) (layer "F.Cu") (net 35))
 (segment (start 106.4 65.7) (end 106.4 55.1) (width 0.2) (layer "F.Cu") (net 35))
 (segment (start 98.415 65.95) (end 98.4 66) (width 0.2) (layer "F.Cu") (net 35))
 (segment (start 98.4 65) (end 98.6 64.8) (width 0.2) (layer "F.Cu") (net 36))
 (segment (start 106 54.9) (end 111 49.9) (width 0.2) (layer "F.Cu") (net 36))
 (segment (start 98.6 64.8) (end 105.9 64.8) (width 0.2) (layer "F.Cu") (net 36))
 (segment (start 105.9 64.8) (end 106 64.7) (width 0.2) (layer "F.Cu") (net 36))
 (segment (start 111 49.9) (end 117.9 49.9) (width 0.2) (layer "F.Cu") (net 36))
 (segment (start 117.9 49.9) (end 120.5 52.5) (width 0.2) (layer "F.Cu") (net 36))
 (segment (start 98.415 64.95) (end 98.4 65) (width 0.2) (layer "F.Cu") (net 36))
 (segment (start 106 64.7) (end 106 54.9) (width 0.2) (layer "F.Cu") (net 36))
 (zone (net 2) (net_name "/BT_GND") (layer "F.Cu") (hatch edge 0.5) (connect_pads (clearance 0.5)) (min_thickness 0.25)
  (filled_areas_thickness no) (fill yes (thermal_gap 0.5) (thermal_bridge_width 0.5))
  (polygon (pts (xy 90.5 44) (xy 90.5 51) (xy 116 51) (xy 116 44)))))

